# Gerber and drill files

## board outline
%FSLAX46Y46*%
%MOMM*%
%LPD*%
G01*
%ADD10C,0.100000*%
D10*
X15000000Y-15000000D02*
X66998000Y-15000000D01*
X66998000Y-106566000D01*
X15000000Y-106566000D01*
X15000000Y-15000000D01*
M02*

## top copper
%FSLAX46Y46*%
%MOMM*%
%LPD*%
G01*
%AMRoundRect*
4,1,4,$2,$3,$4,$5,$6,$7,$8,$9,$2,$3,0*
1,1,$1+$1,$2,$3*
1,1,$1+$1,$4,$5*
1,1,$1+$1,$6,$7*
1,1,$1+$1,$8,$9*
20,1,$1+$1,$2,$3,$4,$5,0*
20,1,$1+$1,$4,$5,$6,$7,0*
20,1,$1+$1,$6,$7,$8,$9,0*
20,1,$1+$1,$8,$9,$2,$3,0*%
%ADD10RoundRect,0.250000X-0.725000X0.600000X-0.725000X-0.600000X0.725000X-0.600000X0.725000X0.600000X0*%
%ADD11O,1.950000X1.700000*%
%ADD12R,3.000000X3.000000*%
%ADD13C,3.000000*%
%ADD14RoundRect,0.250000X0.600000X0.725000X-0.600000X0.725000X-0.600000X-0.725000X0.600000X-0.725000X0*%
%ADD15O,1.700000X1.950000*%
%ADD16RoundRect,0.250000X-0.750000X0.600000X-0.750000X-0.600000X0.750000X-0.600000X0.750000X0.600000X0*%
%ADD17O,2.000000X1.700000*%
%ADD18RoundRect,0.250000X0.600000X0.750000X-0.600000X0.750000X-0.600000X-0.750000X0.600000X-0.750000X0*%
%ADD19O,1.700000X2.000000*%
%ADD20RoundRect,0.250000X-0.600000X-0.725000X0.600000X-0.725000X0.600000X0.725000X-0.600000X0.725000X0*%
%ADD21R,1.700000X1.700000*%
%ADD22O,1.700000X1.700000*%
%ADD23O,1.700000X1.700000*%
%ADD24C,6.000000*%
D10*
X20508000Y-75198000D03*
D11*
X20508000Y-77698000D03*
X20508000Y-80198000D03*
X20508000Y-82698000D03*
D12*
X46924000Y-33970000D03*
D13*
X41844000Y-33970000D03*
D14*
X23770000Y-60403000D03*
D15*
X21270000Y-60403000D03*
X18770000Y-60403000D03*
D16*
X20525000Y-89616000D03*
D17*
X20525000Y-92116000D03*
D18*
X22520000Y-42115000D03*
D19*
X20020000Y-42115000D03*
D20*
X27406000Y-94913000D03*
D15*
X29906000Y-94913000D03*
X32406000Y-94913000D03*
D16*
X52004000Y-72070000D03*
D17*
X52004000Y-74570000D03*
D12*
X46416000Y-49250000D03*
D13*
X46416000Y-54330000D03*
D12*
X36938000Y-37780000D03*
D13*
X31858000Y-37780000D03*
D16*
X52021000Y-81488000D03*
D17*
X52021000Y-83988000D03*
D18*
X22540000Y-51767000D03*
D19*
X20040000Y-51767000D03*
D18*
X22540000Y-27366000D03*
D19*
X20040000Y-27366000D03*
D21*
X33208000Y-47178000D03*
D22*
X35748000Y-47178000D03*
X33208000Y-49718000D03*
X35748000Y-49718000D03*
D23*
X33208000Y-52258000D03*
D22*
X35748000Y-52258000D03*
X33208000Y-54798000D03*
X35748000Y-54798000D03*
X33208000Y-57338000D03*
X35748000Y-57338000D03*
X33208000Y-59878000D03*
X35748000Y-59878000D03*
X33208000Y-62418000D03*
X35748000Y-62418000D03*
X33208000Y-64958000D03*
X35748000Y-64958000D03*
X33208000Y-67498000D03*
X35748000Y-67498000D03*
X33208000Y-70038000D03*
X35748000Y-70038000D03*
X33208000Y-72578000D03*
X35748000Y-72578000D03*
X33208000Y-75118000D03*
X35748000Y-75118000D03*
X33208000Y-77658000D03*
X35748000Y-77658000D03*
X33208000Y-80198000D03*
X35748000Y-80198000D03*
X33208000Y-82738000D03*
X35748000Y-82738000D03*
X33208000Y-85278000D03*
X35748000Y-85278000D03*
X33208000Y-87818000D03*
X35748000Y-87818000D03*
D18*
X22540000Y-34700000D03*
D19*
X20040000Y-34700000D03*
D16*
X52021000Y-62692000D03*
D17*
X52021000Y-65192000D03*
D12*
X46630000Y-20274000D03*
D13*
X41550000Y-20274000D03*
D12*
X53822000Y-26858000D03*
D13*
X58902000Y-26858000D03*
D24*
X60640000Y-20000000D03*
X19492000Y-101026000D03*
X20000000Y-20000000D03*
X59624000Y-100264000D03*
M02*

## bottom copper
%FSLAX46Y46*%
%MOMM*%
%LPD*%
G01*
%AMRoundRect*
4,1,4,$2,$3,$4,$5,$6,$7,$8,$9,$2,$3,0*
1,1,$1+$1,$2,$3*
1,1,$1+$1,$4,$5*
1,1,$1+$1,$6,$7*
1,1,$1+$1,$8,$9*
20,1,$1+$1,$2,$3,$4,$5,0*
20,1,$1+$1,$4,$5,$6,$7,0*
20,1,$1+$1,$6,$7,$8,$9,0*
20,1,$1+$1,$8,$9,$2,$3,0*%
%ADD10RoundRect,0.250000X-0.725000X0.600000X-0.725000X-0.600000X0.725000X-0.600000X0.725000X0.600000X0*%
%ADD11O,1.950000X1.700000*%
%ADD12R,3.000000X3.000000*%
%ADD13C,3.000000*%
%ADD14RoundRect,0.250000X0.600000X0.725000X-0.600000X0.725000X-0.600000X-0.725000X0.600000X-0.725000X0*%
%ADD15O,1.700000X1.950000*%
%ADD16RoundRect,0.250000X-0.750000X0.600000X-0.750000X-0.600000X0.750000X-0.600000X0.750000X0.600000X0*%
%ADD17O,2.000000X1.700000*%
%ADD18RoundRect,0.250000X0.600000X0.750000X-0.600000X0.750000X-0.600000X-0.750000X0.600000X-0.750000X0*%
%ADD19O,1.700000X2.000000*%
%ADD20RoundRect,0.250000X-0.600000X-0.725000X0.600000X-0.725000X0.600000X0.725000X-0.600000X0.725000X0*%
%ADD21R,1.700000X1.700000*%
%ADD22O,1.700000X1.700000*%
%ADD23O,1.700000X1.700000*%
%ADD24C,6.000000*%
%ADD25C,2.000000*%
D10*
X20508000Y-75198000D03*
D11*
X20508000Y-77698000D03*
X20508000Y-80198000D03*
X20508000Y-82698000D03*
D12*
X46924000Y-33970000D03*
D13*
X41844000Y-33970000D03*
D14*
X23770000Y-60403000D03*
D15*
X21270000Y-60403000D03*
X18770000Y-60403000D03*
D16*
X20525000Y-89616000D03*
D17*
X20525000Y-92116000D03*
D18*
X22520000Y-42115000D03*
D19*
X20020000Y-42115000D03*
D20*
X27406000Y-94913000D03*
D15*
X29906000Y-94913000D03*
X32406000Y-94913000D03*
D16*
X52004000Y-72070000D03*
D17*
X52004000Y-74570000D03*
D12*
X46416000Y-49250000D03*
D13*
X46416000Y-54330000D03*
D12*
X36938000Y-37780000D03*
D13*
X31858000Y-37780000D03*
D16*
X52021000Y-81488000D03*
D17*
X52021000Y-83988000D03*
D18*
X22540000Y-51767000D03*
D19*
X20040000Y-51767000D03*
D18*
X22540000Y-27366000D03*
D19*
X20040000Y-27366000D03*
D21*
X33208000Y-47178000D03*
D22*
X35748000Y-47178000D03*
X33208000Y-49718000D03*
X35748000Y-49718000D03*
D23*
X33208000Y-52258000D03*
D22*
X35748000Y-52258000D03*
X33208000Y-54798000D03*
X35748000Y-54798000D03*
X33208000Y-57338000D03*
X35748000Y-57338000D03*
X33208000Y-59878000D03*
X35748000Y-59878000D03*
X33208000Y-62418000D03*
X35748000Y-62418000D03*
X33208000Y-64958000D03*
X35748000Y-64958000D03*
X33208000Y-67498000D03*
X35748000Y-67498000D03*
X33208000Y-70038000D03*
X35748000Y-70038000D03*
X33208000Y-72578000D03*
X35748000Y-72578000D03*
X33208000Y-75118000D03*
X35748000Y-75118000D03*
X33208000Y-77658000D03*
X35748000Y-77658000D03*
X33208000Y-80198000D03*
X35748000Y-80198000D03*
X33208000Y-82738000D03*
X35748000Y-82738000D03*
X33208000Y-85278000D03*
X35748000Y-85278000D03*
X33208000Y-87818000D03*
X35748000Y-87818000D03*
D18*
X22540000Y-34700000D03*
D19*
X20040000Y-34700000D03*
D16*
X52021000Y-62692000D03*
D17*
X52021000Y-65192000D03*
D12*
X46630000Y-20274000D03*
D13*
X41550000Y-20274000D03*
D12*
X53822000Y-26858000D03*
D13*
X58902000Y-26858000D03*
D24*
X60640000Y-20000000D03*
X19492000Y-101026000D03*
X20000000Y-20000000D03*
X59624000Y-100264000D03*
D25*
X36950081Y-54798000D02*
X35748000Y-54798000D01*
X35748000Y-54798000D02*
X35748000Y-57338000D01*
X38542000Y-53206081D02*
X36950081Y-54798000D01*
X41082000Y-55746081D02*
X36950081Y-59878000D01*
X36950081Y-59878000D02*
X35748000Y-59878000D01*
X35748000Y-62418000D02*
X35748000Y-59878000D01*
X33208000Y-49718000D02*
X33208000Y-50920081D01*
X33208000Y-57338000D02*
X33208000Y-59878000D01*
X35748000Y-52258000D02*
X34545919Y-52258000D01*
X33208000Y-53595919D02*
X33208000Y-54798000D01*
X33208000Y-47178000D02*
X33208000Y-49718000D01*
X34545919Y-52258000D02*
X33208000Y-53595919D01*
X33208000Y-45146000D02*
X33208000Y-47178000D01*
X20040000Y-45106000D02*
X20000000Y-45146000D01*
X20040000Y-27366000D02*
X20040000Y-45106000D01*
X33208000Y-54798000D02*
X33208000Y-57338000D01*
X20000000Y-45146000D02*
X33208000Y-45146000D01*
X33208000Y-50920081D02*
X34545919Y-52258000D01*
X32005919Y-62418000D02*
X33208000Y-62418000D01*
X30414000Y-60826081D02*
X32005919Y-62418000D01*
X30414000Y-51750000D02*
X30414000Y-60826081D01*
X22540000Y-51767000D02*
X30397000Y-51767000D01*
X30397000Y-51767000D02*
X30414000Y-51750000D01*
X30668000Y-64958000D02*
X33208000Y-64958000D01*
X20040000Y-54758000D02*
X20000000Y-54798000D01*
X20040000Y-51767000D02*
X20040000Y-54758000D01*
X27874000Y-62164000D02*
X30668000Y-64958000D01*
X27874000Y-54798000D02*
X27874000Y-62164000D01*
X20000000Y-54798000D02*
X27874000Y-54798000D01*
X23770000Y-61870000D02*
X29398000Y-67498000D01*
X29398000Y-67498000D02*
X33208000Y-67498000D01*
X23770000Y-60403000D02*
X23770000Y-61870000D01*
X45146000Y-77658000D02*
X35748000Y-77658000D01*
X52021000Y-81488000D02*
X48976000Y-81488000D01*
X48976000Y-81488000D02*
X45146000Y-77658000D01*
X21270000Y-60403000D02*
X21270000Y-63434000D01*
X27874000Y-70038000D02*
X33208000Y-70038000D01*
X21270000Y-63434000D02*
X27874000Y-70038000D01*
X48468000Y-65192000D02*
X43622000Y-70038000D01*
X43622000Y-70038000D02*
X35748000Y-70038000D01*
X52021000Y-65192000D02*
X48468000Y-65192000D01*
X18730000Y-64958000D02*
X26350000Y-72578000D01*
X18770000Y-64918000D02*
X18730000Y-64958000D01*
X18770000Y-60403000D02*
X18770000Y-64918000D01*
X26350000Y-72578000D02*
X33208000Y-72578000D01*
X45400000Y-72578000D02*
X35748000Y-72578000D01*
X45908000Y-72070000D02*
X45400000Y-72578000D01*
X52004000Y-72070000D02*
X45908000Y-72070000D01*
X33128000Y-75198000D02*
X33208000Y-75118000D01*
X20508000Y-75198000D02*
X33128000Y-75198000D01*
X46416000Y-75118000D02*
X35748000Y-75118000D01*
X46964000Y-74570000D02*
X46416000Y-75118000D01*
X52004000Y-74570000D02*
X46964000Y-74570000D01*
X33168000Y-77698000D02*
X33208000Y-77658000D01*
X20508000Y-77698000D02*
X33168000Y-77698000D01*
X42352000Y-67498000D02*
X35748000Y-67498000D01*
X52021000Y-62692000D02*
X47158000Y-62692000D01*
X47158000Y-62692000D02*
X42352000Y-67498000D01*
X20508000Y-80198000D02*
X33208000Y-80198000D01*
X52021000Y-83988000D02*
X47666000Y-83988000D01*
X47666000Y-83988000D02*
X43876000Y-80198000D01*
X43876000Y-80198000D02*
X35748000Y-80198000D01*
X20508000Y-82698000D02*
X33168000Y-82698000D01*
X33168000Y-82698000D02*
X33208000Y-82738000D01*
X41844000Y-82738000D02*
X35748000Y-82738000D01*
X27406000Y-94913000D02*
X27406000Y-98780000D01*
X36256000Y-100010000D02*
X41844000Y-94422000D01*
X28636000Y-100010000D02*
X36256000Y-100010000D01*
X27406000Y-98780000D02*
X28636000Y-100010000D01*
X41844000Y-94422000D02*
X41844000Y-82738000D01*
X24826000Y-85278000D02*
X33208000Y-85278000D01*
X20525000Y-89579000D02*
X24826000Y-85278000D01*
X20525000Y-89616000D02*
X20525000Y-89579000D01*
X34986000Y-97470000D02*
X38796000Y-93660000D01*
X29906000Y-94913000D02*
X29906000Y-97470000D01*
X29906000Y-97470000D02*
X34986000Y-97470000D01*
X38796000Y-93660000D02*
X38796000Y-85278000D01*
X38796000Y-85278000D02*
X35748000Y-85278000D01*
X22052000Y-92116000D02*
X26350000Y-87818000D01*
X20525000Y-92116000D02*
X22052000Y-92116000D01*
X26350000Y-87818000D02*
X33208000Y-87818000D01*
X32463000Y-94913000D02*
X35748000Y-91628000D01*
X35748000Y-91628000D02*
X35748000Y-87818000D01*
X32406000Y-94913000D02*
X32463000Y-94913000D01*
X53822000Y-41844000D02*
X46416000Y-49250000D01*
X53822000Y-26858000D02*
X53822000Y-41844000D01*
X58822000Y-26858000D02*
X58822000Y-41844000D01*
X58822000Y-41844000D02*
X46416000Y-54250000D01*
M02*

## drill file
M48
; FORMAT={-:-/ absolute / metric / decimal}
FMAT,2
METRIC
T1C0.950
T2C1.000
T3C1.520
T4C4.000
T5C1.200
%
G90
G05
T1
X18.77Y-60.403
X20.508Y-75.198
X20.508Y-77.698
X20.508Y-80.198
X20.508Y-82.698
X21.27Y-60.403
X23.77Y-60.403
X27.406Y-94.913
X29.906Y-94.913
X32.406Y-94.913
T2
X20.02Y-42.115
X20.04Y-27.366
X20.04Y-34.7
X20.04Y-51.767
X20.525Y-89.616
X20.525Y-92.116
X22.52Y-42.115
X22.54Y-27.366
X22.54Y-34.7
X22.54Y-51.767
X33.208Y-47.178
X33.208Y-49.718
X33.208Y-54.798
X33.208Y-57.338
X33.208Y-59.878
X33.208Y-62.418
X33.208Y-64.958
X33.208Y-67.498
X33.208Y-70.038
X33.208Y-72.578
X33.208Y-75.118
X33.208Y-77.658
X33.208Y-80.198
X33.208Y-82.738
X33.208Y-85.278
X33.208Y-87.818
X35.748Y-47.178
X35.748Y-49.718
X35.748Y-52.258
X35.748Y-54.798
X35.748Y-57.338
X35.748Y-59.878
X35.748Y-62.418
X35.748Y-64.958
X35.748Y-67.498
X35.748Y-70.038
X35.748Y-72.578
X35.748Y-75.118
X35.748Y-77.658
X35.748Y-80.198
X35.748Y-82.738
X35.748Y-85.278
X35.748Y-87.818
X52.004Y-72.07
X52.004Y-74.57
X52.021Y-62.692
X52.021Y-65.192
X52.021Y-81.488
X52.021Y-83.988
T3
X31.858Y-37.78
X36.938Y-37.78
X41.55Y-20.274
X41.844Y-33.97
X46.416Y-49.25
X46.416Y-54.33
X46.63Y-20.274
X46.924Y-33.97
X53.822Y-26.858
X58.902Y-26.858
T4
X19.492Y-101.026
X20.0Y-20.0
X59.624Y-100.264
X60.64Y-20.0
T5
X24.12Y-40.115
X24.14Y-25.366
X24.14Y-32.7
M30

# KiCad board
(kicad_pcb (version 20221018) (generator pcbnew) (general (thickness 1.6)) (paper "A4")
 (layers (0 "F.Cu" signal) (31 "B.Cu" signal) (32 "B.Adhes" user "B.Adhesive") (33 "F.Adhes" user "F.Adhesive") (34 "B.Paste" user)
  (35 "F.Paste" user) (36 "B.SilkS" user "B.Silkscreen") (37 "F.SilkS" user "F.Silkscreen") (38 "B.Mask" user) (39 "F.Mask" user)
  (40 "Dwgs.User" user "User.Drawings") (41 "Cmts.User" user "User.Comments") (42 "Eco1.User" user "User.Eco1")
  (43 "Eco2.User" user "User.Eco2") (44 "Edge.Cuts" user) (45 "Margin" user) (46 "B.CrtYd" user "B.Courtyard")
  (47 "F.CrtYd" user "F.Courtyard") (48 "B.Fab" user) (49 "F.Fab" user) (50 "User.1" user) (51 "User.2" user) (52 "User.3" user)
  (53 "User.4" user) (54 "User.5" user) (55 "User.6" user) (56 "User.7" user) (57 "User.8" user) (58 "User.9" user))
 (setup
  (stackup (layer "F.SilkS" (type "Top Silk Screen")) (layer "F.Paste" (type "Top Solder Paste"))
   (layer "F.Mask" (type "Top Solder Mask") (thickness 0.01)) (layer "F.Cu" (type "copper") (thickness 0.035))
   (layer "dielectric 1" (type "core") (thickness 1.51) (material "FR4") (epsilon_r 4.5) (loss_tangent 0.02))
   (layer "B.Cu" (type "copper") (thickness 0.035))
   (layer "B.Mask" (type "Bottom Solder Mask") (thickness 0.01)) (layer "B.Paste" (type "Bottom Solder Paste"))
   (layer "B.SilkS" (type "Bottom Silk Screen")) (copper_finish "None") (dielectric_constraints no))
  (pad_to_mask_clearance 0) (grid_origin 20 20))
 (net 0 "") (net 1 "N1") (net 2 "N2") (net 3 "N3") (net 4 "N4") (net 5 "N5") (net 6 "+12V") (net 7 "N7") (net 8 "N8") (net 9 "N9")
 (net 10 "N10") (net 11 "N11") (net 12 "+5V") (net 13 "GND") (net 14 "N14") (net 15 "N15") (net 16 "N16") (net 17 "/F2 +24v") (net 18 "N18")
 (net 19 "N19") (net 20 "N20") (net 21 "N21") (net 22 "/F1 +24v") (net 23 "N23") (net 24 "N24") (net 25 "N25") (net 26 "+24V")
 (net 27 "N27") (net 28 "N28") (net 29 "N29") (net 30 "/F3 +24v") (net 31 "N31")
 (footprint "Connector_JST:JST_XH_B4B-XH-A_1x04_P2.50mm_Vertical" (layer "F.Cu") (at 20.508 75.198 -90)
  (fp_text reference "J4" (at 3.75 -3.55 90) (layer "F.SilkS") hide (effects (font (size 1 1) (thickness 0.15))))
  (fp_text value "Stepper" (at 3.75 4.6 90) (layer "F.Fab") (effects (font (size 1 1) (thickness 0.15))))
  (pad "1" thru_hole roundrect (at 0 0 270) (size 1.7 1.95) (drill 0.95) (layers "*.Cu" "*.Mask") (roundrect_rratio 0.1470588235)
   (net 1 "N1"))
  (pad "2" thru_hole oval (at 2.5 0 270) (size 1.7 1.95) (drill 0.95) (layers "*.Cu" "*.Mask") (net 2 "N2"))
  (pad "3" thru_hole oval (at 5 0 270) (size 1.7 1.95) (drill 0.95) (layers "*.Cu" "*.Mask") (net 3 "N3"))
  (pad "4" thru_hole oval (at 7.5 0 270) (size 1.7 1.95) (drill 0.95) (layers "*.Cu" "*.Mask") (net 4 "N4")))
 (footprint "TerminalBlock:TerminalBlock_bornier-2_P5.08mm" (layer "F.Cu") (at 46.924 33.97 180)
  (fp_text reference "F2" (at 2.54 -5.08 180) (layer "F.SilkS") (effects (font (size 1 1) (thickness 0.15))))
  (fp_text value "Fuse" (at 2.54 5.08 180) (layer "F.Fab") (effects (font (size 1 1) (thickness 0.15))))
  (pad "1" thru_hole rect (at 0 0 180) (size 3 3) (drill 1.52) (layers "*.Cu" "*.Mask") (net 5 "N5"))
  (pad "2" thru_hole circle (at 5.08 0 180) (size 3 3) (drill 1.52) (layers "*.Cu" "*.Mask") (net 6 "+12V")))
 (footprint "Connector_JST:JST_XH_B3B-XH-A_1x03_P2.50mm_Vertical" (layer "F.Cu") (at 23.77 60.403 180)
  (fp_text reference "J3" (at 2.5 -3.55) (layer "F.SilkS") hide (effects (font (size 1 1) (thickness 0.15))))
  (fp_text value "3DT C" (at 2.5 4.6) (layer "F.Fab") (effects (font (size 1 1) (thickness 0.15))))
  (pad "1" thru_hole roundrect (at 0 0 180) (size 1.7 1.95) (drill 0.95) (layers "*.Cu" "*.Mask") (roundrect_rratio 0.1470588235)
   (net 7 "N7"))
  (pad "2" thru_hole oval (at 2.5 0 180) (size 1.7 1.95) (drill 0.95) (layers "*.Cu" "*.Mask") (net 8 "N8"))
  (pad "3" thru_hole oval (at 5 0 180) (size 1.7 1.95) (drill 0.95) (layers "*.Cu" "*.Mask") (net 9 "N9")))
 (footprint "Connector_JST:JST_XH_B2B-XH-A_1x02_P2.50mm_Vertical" (layer "F.Cu") (at 20.525 89.616 -90)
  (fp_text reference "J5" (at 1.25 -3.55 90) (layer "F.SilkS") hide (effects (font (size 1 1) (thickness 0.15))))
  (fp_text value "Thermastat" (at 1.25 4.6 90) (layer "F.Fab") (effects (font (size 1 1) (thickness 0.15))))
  (pad "1" thru_hole roundrect (at 0 0 270) (size 1.7 2) (drill 1) (layers "*.Cu" "*.Mask") (roundrect_rratio 0.1470588235) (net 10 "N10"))
  (pad "2" thru_hole oval (at 2.5 0 270) (size 1.7 2) (drill 1) (layers "*.Cu" "*.Mask") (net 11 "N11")))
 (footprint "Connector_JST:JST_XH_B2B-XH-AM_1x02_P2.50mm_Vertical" (layer "F.Cu") (at 22.52 42.115 180)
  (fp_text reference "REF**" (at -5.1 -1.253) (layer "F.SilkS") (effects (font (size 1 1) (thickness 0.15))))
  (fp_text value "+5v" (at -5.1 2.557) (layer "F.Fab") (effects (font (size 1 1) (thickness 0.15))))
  (pad "" np_thru_hole circle (at -1.6 2 180) (size 1.2 1.2) (drill 1.2) (layers "F&B.Cu" "*.Mask"))
  (pad "1" thru_hole roundrect (at 0 0 180) (size 1.7 2) (drill 1) (layers "*.Cu" "*.Mask") (roundrect_rratio 0.1470588235) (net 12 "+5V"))
  (pad "2" thru_hole oval (at 2.5 0 180) (size 1.7 2) (drill 1) (layers "*.Cu" "*.Mask") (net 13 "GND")))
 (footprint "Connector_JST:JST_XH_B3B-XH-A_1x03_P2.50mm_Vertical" (layer "F.Cu") (at 27.406 94.913)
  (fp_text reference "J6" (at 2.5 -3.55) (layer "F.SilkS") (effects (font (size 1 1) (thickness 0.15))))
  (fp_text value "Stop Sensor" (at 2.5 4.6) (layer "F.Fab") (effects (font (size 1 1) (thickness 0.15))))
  (pad "1" thru_hole roundrect (at 0 0) (size 1.7 1.95) (drill 0.95) (layers "*.Cu" "*.Mask") (roundrect_rratio 0.1470588235) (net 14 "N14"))
  (pad "2" thru_hole oval (at 2.5 0) (size 1.7 1.95) (drill 0.95) (layers "*.Cu" "*.Mask") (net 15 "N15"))
  (pad "3" thru_hole oval (at 5 0) (size 1.7 1.95) (drill 0.95) (layers "*.Cu" "*.Mask") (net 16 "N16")))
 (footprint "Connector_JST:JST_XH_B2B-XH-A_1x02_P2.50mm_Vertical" (layer "F.Cu") (at 52.004 72.07 -90)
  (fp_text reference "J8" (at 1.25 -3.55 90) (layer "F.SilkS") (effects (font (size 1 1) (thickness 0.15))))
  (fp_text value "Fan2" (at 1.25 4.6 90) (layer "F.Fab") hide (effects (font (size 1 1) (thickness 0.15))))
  (pad "1" thru_hole roundrect (at 0 0 270) (size 1.7 2) (drill 1) (layers "*.Cu" "*.Mask") (roundrect_rratio 0.1470588235)
   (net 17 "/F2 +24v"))
  (pad "2" thru_hole oval (at 2.5 0 270) (size 1.7 2) (drill 1) (layers "*.Cu" "*.Mask") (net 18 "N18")))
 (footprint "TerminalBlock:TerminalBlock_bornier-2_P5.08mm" (layer "F.Cu") (at 46.416 49.25 -90)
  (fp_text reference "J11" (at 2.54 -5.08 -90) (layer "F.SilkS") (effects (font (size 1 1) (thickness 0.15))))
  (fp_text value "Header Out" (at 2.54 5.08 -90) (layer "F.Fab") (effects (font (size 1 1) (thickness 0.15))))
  (pad "1" thru_hole rect (at 0 0 270) (size 3 3) (drill 1.52) (layers "*.Cu" "*.Mask") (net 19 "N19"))
  (pad "2" thru_hole circle (at 5.08 0 270) (size 3 3) (drill 1.52) (layers "*.Cu" "*.Mask") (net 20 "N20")))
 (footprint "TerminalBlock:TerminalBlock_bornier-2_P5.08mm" (layer "F.Cu") (at 36.938 37.78 180)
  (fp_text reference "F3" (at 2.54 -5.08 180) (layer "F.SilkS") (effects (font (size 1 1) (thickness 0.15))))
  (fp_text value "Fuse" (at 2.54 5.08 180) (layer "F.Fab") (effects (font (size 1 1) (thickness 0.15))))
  (pad "1" thru_hole rect (at 0 0 180) (size 3 3) (drill 1.52) (layers "*.Cu" "*.Mask") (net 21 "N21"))
  (pad "2" thru_hole circle (at 5.08 0 180) (size 3 3) (drill 1.52) (layers "*.Cu" "*.Mask") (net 12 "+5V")))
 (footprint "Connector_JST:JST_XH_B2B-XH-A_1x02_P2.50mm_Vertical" (layer "F.Cu") (at 52.021 81.488 -90)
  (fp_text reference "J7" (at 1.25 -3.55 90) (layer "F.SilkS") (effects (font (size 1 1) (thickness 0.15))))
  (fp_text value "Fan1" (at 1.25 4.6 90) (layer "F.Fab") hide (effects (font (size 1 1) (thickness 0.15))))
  (pad "1" thru_hole roundrect (at 0 0 270) (size 1.7 2) (drill 1) (layers "*.Cu" "*.Mask") (roundrect_rratio 0.1470588235)
   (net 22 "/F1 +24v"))
  (pad "2" thru_hole oval (at 2.5 0 270) (size 1.7 2) (drill 1) (layers "*.Cu" "*.Mask") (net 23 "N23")))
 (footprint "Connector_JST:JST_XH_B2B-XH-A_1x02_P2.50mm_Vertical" (layer "F.Cu") (at 22.54 51.767 180)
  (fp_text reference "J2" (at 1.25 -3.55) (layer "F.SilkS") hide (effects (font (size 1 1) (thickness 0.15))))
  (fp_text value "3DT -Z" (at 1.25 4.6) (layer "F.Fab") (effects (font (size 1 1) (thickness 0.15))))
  (pad "1" thru_hole roundrect (at 0 0 180) (size 1.7 2) (drill 1) (layers "*.Cu" "*.Mask") (roundrect_rratio 0.1470588235) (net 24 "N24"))
  (pad "2" thru_hole oval (at 2.5 0 180) (size 1.7 2) (drill 1) (layers "*.Cu" "*.Mask") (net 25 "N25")))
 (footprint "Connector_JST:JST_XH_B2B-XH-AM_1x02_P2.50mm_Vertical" (layer "F.Cu") (at 22.54 27.366 180)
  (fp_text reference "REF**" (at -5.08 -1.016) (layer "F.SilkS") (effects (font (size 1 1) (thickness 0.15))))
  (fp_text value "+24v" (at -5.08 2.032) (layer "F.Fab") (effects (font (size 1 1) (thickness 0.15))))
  (pad "" np_thru_hole circle (at -1.6 2 180) (size 1.2 1.2) (drill 1.2) (layers "*.Cu" "*.Mask"))
  (pad "1" thru_hole roundrect (at 0 0 180) (size 1.7 2) (drill 1) (layers "*.Cu" "*.Mask") (roundrect_rratio 0.1470588235) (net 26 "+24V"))
  (pad "2" thru_hole oval (at 2.5 0 180) (size 1.7 2) (drill 1) (layers "*.Cu" "*.Mask") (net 13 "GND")))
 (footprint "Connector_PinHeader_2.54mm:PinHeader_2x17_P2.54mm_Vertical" (layer "F.Cu") (at 33.208 47.178)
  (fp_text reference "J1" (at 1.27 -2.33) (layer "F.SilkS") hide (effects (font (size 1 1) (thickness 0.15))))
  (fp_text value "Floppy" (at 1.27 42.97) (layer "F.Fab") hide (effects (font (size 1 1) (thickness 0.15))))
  (pad "1" thru_hole rect (at 0 0) (size 1.7 1.7) (drill 1) (layers "*.Cu" "*.Mask") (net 13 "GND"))
  (pad "2" thru_hole oval (at 2.54 0) (size 1.7 1.7) (drill 1) (layers "*.Cu" "*.Mask") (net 21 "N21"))
  (pad "3" thru_hole oval (at 0 2.54) (size 1.7 1.7) (drill 1) (layers "*.Cu" "*.Mask") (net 13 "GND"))
  (pad "4" thru_hole oval (at 2.54 2.54) (size 1.7 1.7) (drill 1) (layers "*.Cu" "*.Mask") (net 21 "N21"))
  (pad "5" smd oval (at 0 5.08) (size 1.7 1.7) (layers "*.Cu" "*.Mask") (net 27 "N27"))
  (pad "6" thru_hole oval (at 2.54 5.08) (size 1.7 1.7) (drill 1) (layers "*.Cu" "*.Mask") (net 13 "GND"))
  (pad "7" thru_hole oval (at 0 7.62) (size 1.7 1.7) (drill 1) (layers "*.Cu" "*.Mask") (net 13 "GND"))
  (pad "8" thru_hole oval (at 2.54 7.62) (size 1.7 1.7) (drill 1) (layers "*.Cu" "*.Mask") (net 5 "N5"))
  (pad "9" thru_hole oval (at 0 10.16) (size 1.7 1.7) (drill 1) (layers "*.Cu" "*.Mask") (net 13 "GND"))
  (pad "10" thru_hole oval (at 2.54 10.16) (size 1.7 1.7) (drill 1) (layers "*.Cu" "*.Mask") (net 5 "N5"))
  (pad "11" thru_hole oval (at 0 12.7) (size 1.7 1.7) (drill 1) (layers "*.Cu" "*.Mask") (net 13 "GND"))
  (pad "12" thru_hole oval (at 2.54 12.7) (size 1.7 1.7) (drill 1) (layers "*.Cu" "*.Mask") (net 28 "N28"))
  (pad "13" thru_hole oval (at 0 15.24) (size 1.7 1.7) (drill 1) (layers "*.Cu" "*.Mask") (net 24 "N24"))
  (pad "14" thru_hole oval (at 2.54 15.24) (size 1.7 1.7) (drill 1) (layers "*.Cu" "*.Mask") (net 28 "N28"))
  (pad "15" thru_hole oval (at 0 17.78) (size 1.7 1.7) (drill 1) (layers "*.Cu" "*.Mask") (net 25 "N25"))
  (pad "16" thru_hole oval (at 2.54 17.78) (size 1.7 1.7) (drill 1) (layers "*.Cu" "*.Mask") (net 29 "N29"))
  (pad "17" thru_hole oval (at 0 20.32) (size 1.7 1.7) (drill 1) (layers "*.Cu" "*.Mask") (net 7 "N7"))
  (pad "18" thru_hole oval (at 2.54 20.32) (size 1.7 1.7) (drill 1) (layers "*.Cu" "*.Mask") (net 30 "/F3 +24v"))
  (pad "19" thru_hole oval (at 0 22.86) (size 1.7 1.7) (drill 1) (layers "*.Cu" "*.Mask") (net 8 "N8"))
  (pad "20" thru_hole oval (at 2.54 22.86) (size 1.7 1.7) (drill 1) (layers "*.Cu" "*.Mask") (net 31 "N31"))
  (pad "21" thru_hole oval (at 0 25.4) (size 1.7 1.7) (drill 1) (layers "*.Cu" "*.Mask") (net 9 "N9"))
  (pad "22" thru_hole oval (at 2.54 25.4) (size 1.7 1.7) (drill 1) (layers "*.Cu" "*.Mask") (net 17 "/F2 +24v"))
  (pad "23" thru_hole oval (at 0 27.94) (size 1.7 1.7) (drill 1) (layers "*.Cu" "*.Mask") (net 1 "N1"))
  (pad "24" thru_hole oval (at 2.54 27.94) (size 1.7 1.7) (drill 1) (layers "*.Cu" "*.Mask") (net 18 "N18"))
  (pad "25" thru_hole oval (at 0 30.48) (size 1.7 1.7) (drill 1) (layers "*.Cu" "*.Mask") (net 2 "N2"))
  (pad "26" thru_hole oval (at 2.54 30.48) (size 1.7 1.7) (drill 1) (layers "*.Cu" "*.Mask") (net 22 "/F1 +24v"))
  (pad "27" thru_hole oval (at 0 33.02) (size 1.7 1.7) (drill 1) (layers "*.Cu" "*.Mask") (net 3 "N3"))
  (pad "28" thru_hole oval (at 2.54 33.02) (size 1.7 1.7) (drill 1) (layers "*.Cu" "*.Mask") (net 23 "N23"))
  (pad "29" thru_hole oval (at 0 35.56) (size 1.7 1.7) (drill 1) (layers "*.Cu" "*.Mask") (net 4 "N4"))
  (pad "30" thru_hole oval (at 2.54 35.56) (size 1.7 1.7) (drill 1) (layers "*.Cu" "*.Mask") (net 14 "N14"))
  (pad "31" thru_hole oval (at 0 38.1) (size 1.7 1.7) (drill 1) (layers "*.Cu" "*.Mask") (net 10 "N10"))
  (pad "32" thru_hole oval (at 2.54 38.1) (size 1.7 1.7) (drill 1) (layers "*.Cu" "*.Mask") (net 15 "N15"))
  (pad "33" thru_hole oval (at 0 40.64) (size 1.7 1.7) (drill 1) (layers "*.Cu" "*.Mask") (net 11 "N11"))
  (pad "34" thru_hole oval (at 2.54 40.64) (size 1.7 1.7) (drill 1) (layers "*.Cu" "*.Mask") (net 16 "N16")))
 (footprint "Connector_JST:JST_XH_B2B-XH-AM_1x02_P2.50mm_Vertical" (layer "F.Cu") (at 22.54 34.7 180)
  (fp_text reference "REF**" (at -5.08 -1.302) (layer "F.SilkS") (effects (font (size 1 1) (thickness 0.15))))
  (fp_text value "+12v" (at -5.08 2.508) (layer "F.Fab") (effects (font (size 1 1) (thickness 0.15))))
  (pad "" np_thru_hole circle (at -1.6 2 180) (size 1.2 1.2) (drill 1.2) (layers "F&B.Cu" "*.Mask"))
  (pad "1" thru_hole roundrect (at 0 0 180) (size 1.7 2) (drill 1) (layers "*.Cu" "*.Mask") (roundrect_rratio 0.1470588235) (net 6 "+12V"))
  (pad "2" thru_hole oval (at 2.5 0 180) (size 1.7 2) (drill 1) (layers "*.Cu" "*.Mask") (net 13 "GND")))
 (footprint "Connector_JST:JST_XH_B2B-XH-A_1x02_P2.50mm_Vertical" (layer "F.Cu") (at 52.021 62.692 -90)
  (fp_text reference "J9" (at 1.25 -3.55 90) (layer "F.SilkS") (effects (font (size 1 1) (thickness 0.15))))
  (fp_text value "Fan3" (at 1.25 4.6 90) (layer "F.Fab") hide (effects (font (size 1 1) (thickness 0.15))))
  (pad "1" thru_hole roundrect (at 0 0 270) (size 1.7 2) (drill 1) (layers "*.Cu" "*.Mask") (roundrect_rratio 0.1470588235)
   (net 30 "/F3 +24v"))
  (pad "2" thru_hole oval (at 2.5 0 270) (size 1.7 2) (drill 1) (layers "*.Cu" "*.Mask") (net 31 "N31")))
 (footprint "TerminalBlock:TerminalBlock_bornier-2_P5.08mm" (layer "F.Cu") (at 46.63 20.274 180)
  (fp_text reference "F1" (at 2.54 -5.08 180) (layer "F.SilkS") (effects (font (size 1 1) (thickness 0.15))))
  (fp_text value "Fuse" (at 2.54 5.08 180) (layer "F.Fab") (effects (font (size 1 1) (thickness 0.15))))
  (pad "1" thru_hole rect (at 0 0 180) (size 3 3) (drill 1.52) (layers "*.Cu" "*.Mask") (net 28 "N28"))
  (pad "2" thru_hole circle (at 5.08 0 180) (size 3 3) (drill 1.52) (layers "*.Cu" "*.Mask") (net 26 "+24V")))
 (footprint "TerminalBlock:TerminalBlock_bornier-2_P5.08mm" (layer "F.Cu") (at 53.822 26.858)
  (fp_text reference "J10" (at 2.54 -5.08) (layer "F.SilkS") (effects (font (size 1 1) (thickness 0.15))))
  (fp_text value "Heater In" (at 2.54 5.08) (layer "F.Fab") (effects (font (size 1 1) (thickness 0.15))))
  (pad "1" thru_hole rect (at 0 0) (size 3 3) (drill 1.52) (layers "*.Cu" "*.Mask") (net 19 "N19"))
  (pad "2" thru_hole circle (at 5.08 0) (size 3 3) (drill 1.52) (layers "*.Cu" "*.Mask") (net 20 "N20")))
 (gr_rect (start 15 15) (end 66.998 106.566) (stroke (width 0.1) (type default)) (fill none) (layer "Edge.Cuts"))
 (via (at 60.64 20) (size 6) (drill 4) (layers "F.Cu" "B.Cu") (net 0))
 (via (at 19.492 101.026) (size 6) (drill 4) (layers "F.Cu" "B.Cu") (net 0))
 (via (at 20 20) (size 6) (drill 4) (layers "F.Cu" "B.Cu") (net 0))
 (via (at 59.624 100.264) (size 6) (drill 4) (layers "F.Cu" "B.Cu") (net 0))
 (segment (start 36.950081 54.798) (end 35.748 54.798) (width 2) (layer "B.Cu") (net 5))
 (segment (start 35.748 54.798) (end 35.748 57.338) (width 2) (layer "B.Cu") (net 5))
 (segment (start 38.542 53.206081) (end 36.950081 54.798) (width 2) (layer "B.Cu") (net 5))
 (segment (start 41.082 55.746081) (end 36.950081 59.878) (width 2) (layer "B.Cu") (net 28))
 (segment (start 36.950081 59.878) (end 35.748 59.878) (width 2) (layer "B.Cu") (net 28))
 (segment (start 35.748 62.418) (end 35.748 59.878) (width 2) (layer "B.Cu") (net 28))
 (segment (start 33.208 49.718) (end 33.208 50.920081) (width 2) (layer "B.Cu") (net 13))
 (segment (start 33.208 57.338) (end 33.208 59.878) (width 2) (layer "B.Cu") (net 13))
 (segment (start 35.748 52.258) (end 34.545919 52.258) (width 2) (layer "B.Cu") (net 13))
 (segment (start 33.208 53.595919) (end 33.208 54.798) (width 2) (layer "B.Cu") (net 13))
 (segment (start 33.208 47.178) (end 33.208 49.718) (width 2) (layer "B.Cu") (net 13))
 (segment (start 34.545919 52.258) (end 33.208 53.595919) (width 2) (layer "B.Cu") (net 13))
 (segment (start 33.208 45.146) (end 33.208 47.178) (width 2) (layer "B.Cu") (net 13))
 (segment (start 20.04 45.106) (end 20 45.146) (width 2) (layer "B.Cu") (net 13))
 (segment (start 20.04 27.366) (end 20.04 45.106) (width 2) (layer "B.Cu") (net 13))
 (segment (start 33.208 54.798) (end 33.208 57.338) (width 2) (layer "B.Cu") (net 13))
 (segment (start 20 45.146) (end 33.208 45.146) (width 2) (layer "B.Cu") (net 13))
 (segment (start 33.208 50.920081) (end 34.545919 52.258) (width 2) (layer "B.Cu") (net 13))
 (segment (start 32.005919 62.418) (end 33.208 62.418) (width 2) (layer "B.Cu") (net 24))
 (segment (start 30.414 60.826081) (end 32.005919 62.418) (width 2) (layer "B.Cu") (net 24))
 (segment (start 30.414 51.75) (end 30.414 60.826081) (width 2) (layer "B.Cu") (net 24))
 (segment (start 22.54 51.767) (end 30.397 51.767) (width 2) (layer "B.Cu") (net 24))
 (segment (start 30.397 51.767) (end 30.414 51.75) (width 2) (layer "B.Cu") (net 24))
 (segment (start 30.668 64.958) (end 33.208 64.958) (width 2) (layer "B.Cu") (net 25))
 (segment (start 20.04 54.758) (end 20 54.798) (width 2) (layer "B.Cu") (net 25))
 (segment (start 20.04 51.767) (end 20.04 54.758) (width 2) (layer "B.Cu") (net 25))
 (segment (start 27.874 62.164) (end 30.668 64.958) (width 2) (layer "B.Cu") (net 25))
 (segment (start 27.874 54.798) (end 27.874 62.164) (width 2) (layer "B.Cu") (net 25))
 (segment (start 20 54.798) (end 27.874 54.798) (width 2) (layer "B.Cu") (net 25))
 (segment (start 23.77 61.87) (end 29.398 67.498) (width 2) (layer "B.Cu") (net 7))
 (segment (start 29.398 67.498) (end 33.208 67.498) (width 2) (layer "B.Cu") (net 7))
 (segment (start 23.77 60.403) (end 23.77 61.87) (width 2) (layer "B.Cu") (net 7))
 (segment (start 45.146 77.658) (end 35.748 77.658) (width 2) (layer "B.Cu") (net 22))
 (segment (start 52.021 81.488) (end 48.976 81.488) (width 2) (layer "B.Cu") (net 22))
 (segment (start 48.976 81.488) (end 45.146 77.658) (width 2) (layer "B.Cu") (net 22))
 (segment (start 21.27 60.403) (end 21.27 63.434) (width 2) (layer "B.Cu") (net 8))
 (segment (start 27.874 70.038) (end 33.208 70.038) (width 2) (layer "B.Cu") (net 8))
 (segment (start 21.27 63.434) (end 27.874 70.038) (width 2) (layer "B.Cu") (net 8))
 (segment (start 48.468 65.192) (end 43.622 70.038) (width 2) (layer "B.Cu") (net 31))
 (segment (start 43.622 70.038) (end 35.748 70.038) (width 2) (layer "B.Cu") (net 31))
 (segment (start 52.021 65.192) (end 48.468 65.192) (width 2) (layer "B.Cu") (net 31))
 (segment (start 18.73 64.958) (end 26.35 72.578) (width 2) (layer "B.Cu") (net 9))
 (segment (start 18.77 64.918) (end 18.73 64.958) (width 2) (layer "B.Cu") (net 9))
 (segment (start 18.77 60.403) (end 18.77 64.918) (width 2) (layer "B.Cu") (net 9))
 (segment (start 26.35 72.578) (end 33.208 72.578) (width 2) (layer "B.Cu") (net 9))
 (segment (start 45.4 72.578) (end 35.748 72.578) (width 2) (layer "B.Cu") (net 17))
 (segment (start 45.908 72.07) (end 45.4 72.578) (width 2) (layer "B.Cu") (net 17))
 (segment (start 52.004 72.07) (end 45.908 72.07) (width 2) (layer "B.Cu") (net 17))
 (segment (start 33.128 75.198) (end 33.208 75.118) (width 2) (layer "B.Cu") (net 1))
 (segment (start 20.508 75.198) (end 33.128 75.198) (width 2) (layer "B.Cu") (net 1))
 (segment (start 46.416 75.118) (end 35.748 75.118) (width 2) (layer "B.Cu") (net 18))
 (segment (start 46.964 74.57) (end 46.416 75.118) (width 2) (layer "B.Cu") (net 18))
 (segment (start 52.004 74.57) (end 46.964 74.57) (width 2) (layer "B.Cu") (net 18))
 (segment (start 33.168 77.698) (end 33.208 77.658) (width 2) (layer "B.Cu") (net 2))
 (segment (start 20.508 77.698) (end 33.168 77.698) (width 2) (layer "B.Cu") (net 2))
 (segment (start 42.352 67.498) (end 35.748 67.498) (width 2) (layer "B.Cu") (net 30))
 (segment (start 52.021 62.692) (end 47.158 62.692) (width 2) (layer "B.Cu") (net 30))
 (segment (start 47.158 62.692) (end 42.352 67.498) (width 2) (layer "B.Cu") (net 30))
 (segment (start 20.508 80.198) (end 33.208 80.198) (width 2) (layer "B.Cu") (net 3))
 (segment (start 52.021 83.988) (end 47.666 83.988) (width 2) (layer "B.Cu") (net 23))
 (segment (start 47.666 83.988) (end 43.876 80.198) (width 2) (layer "B.Cu") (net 23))
 (segment (start 43.876 80.198) (end 35.748 80.198) (width 2) (layer "B.Cu") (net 23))
 (segment (start 20.508 82.698) (end 33.168 82.698) (width 2) (layer "B.Cu") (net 4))
 (segment (start 33.168 82.698) (end 33.208 82.738) (width 2) (layer "B.Cu") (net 4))
 (segment (start 41.844 82.738) (end 35.748 82.738) (width 2) (layer "B.Cu") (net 14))
 (segment (start 27.406 94.913) (end 27.406 98.78) (width 2) (layer "B.Cu") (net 14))
 (segment (start 36.256 100.01) (end 41.844 94.422) (width 2) (layer "B.Cu") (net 14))
 (segment (start 28.636 100.01) (end 36.256 100.01) (width 2) (layer "B.Cu") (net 14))
 (segment (start 27.406 98.78) (end 28.636 100.01) (width 2) (layer "B.Cu") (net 14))
 (segment (start 41.844 94.422) (end 41.844 82.738) (width 2) (layer "B.Cu") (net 14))
 (segment (start 24.826 85.278) (end 33.208 85.278) (width 2) (layer "B.Cu") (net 10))
 (segment (start 20.525 89.579) (end 24.826 85.278) (width 2) (layer "B.Cu") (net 10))
 (segment (start 20.525 89.616) (end 20.525 89.579) (width 2) (layer "B.Cu") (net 10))
 (segment (start 34.986 97.47) (end 38.796 93.66) (width 2) (layer "B.Cu") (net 15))
 (segment (start 29.906 94.913) (end 29.906 97.47) (width 2) (layer "B.Cu") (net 15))
 (segment (start 29.906 97.47) (end 34.986 97.47) (width 2) (layer "B.Cu") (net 15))
 (segment (start 38.796 93.66) (end 38.796 85.278) (width 2) (layer "B.Cu") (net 15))
 (segment (start 38.796 85.278) (end 35.748 85.278) (width 2) (layer "B.Cu") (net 15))
 (segment (start 22.052 92.116) (end 26.35 87.818) (width 2) (layer "B.Cu") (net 11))
 (segment (start 20.525 92.116) (end 22.052 92.116) (width 2) (layer "B.Cu") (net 11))
 (segment (start 26.35 87.818) (end 33.208 87.818) (width 2) (layer "B.Cu") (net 11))
 (segment (start 32.463 94.913) (end 35.748 91.628) (width 2) (layer "B.Cu") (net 16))
 (segment (start 35.748 91.628) (end 35.748 87.818) (width 2) (layer "B.Cu") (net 16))
 (segment (start 32.406 94.913) (end 32.463 94.913) (width 2) (layer "B.Cu") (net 16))
 (segment (start 53.822 41.844) (end 46.416 49.25) (width 2) (layer "B.Cu") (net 19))
 (segment (start 53.822 26.858) (end 53.822 41.844) (width 2) (layer "B.Cu") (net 19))
 (segment (start 58.822 26.858) (end 58.822 41.844) (width 2) (layer "B.Cu") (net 20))
 (segment (start 58.822 41.844) (end 46.416 54.25) (width 2) (layer "B.Cu") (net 20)))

